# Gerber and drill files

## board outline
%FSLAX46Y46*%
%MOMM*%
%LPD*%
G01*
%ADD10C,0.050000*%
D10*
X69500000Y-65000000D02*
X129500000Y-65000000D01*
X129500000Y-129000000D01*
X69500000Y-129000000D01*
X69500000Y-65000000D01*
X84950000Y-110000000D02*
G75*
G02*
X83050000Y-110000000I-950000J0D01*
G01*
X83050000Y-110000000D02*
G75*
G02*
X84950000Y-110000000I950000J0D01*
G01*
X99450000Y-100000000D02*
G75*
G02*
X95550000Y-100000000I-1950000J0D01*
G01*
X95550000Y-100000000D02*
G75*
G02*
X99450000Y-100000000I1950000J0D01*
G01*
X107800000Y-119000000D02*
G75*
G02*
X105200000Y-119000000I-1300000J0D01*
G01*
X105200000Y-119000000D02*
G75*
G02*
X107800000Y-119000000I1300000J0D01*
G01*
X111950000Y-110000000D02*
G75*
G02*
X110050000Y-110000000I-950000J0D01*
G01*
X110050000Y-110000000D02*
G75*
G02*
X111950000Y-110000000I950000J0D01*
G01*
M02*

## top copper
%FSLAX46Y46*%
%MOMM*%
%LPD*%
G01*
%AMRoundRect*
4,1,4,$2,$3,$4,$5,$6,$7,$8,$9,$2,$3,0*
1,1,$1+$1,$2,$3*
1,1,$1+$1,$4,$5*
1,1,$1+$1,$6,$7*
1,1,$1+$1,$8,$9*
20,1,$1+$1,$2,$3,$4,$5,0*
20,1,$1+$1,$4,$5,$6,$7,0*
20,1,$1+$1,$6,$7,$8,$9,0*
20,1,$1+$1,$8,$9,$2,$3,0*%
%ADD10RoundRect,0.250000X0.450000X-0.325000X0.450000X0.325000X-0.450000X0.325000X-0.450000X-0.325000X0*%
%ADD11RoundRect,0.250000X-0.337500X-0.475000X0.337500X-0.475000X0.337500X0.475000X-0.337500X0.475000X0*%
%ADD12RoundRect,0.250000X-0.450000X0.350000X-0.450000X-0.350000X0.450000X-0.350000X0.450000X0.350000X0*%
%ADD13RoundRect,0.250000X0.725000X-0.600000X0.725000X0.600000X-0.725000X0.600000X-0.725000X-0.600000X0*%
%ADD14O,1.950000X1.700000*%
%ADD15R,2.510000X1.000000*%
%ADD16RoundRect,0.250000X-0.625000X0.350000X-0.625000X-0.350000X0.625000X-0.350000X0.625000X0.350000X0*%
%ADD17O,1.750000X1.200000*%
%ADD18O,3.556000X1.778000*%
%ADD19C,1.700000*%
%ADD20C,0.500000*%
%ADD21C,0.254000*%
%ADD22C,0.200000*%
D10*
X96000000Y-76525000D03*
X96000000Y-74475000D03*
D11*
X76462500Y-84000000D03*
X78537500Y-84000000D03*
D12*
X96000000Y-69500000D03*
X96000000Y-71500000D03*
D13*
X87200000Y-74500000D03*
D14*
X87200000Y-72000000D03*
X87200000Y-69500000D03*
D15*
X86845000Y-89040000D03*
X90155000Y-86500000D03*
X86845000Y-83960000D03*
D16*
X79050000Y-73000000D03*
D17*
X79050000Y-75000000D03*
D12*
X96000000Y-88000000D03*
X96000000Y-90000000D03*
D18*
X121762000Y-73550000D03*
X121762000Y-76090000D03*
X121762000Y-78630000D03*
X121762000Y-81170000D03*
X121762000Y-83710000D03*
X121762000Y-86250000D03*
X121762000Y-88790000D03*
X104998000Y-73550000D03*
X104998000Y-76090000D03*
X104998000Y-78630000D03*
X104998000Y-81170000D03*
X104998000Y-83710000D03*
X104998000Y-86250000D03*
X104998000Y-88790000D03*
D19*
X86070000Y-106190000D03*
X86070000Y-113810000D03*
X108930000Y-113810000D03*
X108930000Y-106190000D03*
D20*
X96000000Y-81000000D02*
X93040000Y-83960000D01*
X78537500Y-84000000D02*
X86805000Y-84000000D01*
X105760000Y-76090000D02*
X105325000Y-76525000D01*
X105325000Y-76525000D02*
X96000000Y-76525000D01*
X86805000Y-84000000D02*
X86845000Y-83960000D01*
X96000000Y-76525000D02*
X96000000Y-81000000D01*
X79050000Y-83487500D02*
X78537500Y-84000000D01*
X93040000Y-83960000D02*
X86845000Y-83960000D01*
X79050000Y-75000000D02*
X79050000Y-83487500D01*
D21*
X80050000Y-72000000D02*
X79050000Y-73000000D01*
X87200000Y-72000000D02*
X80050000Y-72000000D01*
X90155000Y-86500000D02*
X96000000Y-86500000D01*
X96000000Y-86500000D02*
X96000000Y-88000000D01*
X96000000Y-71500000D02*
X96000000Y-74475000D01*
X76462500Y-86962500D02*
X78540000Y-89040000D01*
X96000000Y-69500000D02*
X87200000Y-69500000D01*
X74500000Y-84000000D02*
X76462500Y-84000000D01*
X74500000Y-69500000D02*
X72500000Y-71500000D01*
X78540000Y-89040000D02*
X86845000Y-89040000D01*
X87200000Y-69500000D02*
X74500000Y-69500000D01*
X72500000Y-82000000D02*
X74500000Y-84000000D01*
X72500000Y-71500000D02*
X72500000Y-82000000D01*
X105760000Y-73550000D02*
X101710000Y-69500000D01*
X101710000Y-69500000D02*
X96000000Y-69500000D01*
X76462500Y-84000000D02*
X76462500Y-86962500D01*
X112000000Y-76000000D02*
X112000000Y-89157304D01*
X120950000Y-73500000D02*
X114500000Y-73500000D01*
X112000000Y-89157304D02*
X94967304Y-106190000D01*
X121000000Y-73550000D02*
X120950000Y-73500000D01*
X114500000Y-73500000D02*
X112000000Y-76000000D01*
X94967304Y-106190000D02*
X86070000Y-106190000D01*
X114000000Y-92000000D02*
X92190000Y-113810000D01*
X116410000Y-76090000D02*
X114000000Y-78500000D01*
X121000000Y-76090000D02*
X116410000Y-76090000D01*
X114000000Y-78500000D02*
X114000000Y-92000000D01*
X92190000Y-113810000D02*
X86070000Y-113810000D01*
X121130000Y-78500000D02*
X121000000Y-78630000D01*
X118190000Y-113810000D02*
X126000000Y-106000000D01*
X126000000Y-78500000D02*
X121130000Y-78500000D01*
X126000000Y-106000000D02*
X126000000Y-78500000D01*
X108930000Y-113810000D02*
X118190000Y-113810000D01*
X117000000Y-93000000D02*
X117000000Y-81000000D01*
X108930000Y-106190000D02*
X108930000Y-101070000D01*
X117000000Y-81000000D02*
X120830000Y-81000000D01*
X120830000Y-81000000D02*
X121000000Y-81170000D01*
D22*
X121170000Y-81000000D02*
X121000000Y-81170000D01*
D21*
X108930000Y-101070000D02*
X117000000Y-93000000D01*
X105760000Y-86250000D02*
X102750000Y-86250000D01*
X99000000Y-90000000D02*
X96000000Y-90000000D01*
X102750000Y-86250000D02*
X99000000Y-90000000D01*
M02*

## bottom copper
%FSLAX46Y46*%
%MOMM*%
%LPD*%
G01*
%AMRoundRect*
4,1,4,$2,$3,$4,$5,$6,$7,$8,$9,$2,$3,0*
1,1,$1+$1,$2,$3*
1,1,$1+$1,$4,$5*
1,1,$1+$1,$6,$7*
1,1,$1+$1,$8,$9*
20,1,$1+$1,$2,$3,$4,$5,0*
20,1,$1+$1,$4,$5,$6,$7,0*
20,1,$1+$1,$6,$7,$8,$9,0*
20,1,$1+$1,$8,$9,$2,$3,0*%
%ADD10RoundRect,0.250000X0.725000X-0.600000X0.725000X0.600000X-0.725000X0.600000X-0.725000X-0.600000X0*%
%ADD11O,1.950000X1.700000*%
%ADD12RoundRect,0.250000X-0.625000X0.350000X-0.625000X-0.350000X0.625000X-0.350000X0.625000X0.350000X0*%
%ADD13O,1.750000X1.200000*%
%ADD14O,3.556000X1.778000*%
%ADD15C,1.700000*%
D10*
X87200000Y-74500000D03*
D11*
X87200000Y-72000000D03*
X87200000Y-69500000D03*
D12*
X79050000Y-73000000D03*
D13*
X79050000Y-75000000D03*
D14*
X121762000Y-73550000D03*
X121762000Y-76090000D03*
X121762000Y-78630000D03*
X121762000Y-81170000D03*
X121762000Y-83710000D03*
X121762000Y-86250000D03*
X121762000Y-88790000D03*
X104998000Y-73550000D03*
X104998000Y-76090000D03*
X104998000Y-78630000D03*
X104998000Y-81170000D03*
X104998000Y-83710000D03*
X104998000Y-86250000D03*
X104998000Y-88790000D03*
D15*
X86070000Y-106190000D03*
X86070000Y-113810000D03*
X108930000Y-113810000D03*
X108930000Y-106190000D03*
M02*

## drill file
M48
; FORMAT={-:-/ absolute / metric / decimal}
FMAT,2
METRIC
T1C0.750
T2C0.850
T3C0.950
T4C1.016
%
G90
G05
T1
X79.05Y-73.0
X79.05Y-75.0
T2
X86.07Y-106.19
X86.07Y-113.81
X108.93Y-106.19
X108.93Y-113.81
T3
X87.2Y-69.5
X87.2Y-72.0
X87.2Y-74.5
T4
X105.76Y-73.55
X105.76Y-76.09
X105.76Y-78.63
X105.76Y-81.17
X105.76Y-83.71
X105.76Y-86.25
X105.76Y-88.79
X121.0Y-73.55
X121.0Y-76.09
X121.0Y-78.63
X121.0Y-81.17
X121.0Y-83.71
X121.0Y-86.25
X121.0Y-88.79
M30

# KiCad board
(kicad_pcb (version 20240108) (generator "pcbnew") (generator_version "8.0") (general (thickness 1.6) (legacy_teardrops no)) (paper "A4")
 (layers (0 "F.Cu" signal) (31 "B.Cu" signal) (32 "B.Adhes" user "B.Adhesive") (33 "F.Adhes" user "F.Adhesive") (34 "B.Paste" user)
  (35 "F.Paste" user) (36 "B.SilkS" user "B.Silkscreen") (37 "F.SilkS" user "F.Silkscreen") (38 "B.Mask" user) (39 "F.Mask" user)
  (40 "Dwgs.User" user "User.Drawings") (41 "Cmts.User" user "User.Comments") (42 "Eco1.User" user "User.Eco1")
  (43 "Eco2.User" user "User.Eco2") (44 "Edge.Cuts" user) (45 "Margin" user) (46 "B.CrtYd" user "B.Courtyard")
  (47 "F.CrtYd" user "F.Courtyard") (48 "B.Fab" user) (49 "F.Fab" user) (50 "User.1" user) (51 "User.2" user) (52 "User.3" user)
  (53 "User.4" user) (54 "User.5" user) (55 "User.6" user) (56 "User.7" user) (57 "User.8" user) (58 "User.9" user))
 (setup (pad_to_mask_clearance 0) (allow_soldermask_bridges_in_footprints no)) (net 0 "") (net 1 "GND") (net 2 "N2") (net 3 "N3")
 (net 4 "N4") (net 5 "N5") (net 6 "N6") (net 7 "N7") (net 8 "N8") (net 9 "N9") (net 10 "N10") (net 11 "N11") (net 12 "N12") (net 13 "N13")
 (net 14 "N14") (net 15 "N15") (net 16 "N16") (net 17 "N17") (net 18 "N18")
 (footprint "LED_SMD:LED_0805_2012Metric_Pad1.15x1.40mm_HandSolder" (layer "F.Cu") (at 96 75.5 90)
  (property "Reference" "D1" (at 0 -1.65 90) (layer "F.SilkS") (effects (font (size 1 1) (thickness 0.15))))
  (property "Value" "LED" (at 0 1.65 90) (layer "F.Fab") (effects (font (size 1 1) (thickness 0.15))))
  (pad "1" smd roundrect (at -1.025 0 90) (size 1.15 1.4) (layers "F.Cu" "F.Paste" "F.Mask") (roundrect_rratio 0.217391) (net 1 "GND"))
  (pad "2" smd roundrect (at 1.025 0 90) (size 1.15 1.4) (layers "F.Cu" "F.Paste" "F.Mask") (roundrect_rratio 0.217391) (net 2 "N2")))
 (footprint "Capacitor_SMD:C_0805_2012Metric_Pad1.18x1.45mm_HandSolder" (layer "F.Cu") (at 77.5 84)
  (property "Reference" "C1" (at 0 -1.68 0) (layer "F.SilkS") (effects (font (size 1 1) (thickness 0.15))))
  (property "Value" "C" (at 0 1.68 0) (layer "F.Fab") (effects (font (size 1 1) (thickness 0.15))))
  (pad "1" smd roundrect (at -1.0375 0) (size 1.175 1.45) (layers "F.Cu" "F.Paste" "F.Mask") (roundrect_rratio 0.212766) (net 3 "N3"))
  (pad "2" smd roundrect (at 1.0375 0) (size 1.175 1.45) (layers "F.Cu" "F.Paste" "F.Mask") (roundrect_rratio 0.212766) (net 1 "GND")))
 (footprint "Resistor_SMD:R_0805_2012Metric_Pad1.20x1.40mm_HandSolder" (layer "F.Cu") (at 96 70.5 -90)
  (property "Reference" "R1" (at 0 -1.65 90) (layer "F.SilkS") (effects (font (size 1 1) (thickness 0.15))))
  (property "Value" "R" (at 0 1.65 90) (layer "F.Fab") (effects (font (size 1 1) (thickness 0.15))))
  (pad "1" smd roundrect (at -1 0 270) (size 1.2 1.4) (layers "F.Cu" "F.Paste" "F.Mask") (roundrect_rratio 0.208333) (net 3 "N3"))
  (pad "2" smd roundrect (at 1 0 270) (size 1.2 1.4) (layers "F.Cu" "F.Paste" "F.Mask") (roundrect_rratio 0.208333) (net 2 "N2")))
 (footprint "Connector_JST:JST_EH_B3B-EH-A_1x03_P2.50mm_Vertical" (layer "F.Cu") (at 87.2 74.5 90)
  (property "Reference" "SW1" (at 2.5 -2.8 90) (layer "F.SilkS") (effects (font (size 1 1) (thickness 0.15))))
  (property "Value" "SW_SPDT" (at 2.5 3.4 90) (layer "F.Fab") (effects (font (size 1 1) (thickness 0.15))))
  (pad "1" thru_hole roundrect (at 0 0 90) (size 1.7 1.95) (drill 0.95) (layers "*.Cu" "*.Mask") (remove_unused_layers no)
   (roundrect_rratio 0.147059) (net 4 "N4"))
  (pad "2" thru_hole oval (at 2.5 0 90) (size 1.7 1.95) (drill 0.95) (layers "*.Cu" "*.Mask") (remove_unused_layers no) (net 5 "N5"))
  (pad "3" thru_hole oval (at 5 0 90) (size 1.7 1.95) (drill 0.95) (layers "*.Cu" "*.Mask") (remove_unused_layers no) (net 3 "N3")))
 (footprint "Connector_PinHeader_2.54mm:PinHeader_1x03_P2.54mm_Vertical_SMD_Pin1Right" (layer "F.Cu") (at 88.5 86.5 180)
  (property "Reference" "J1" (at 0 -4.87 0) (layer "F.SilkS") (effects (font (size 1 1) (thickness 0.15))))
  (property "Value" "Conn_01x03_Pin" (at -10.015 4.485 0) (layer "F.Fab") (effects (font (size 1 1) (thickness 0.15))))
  (pad "1" smd rect (at 1.655 -2.54 180) (size 2.51 1) (layers "F.Cu" "F.Paste" "F.Mask") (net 3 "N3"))
  (pad "2" smd rect (at -1.655 0 180) (size 2.51 1) (layers "F.Cu" "F.Paste" "F.Mask") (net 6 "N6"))
  (pad "3" smd rect (at 1.655 2.54 180) (size 2.51 1) (layers "F.Cu" "F.Paste" "F.Mask") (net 1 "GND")))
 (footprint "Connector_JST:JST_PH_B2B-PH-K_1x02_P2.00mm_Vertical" (layer "F.Cu") (at 79.05 73 -90)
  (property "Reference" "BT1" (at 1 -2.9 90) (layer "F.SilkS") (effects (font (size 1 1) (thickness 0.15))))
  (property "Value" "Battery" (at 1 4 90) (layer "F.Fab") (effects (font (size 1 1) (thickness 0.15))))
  (pad "1" thru_hole roundrect (at 0 0 270) (size 1.2 1.75) (drill 0.75) (layers "*.Cu" "*.Mask") (remove_unused_layers no)
   (roundrect_rratio 0.208333) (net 5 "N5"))
  (pad "2" thru_hole oval (at 2 0 270) (size 1.2 1.75) (drill 0.75) (layers "*.Cu" "*.Mask") (remove_unused_layers no) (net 1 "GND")))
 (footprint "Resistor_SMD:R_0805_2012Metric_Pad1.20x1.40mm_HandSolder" (layer "F.Cu") (at 96 89 -90)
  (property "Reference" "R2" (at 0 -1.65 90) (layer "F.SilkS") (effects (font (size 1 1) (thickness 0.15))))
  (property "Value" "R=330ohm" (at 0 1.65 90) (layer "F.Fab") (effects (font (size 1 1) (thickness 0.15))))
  (pad "1" smd roundrect (at -1 0 270) (size 1.2 1.4) (layers "F.Cu" "F.Paste" "F.Mask") (roundrect_rratio 0.208333) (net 6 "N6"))
  (pad "2" smd roundrect (at 1 0 270) (size 1.2 1.4) (layers "F.Cu" "F.Paste" "F.Mask") (roundrect_rratio 0.208333) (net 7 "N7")))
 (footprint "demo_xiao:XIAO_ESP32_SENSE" (layer "B.Cu") (at 113.38 81.17 180)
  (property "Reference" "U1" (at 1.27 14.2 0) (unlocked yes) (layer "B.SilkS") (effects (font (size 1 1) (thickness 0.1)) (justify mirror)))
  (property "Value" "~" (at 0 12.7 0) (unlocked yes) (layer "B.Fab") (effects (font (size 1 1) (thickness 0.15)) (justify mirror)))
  (pad "1" thru_hole oval (at -7.62 7.62 180) (size 3.556 1.778) (drill 1.016 (offset -0.762 0)) (layers "*.Cu" "*.Mask")
   (remove_unused_layers no) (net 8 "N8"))
  (pad "2" thru_hole oval (at -7.62 5.08 180) (size 3.556 1.778) (drill 1.016 (offset -0.762 0)) (layers "*.Cu" "*.Mask")
   (remove_unused_layers no) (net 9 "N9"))
  (pad "3" thru_hole oval (at -7.62 2.54 180) (size 3.556 1.778) (drill 1.016 (offset -0.762 0)) (layers "*.Cu" "*.Mask")
   (remove_unused_layers no) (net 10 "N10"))
  (pad "4" thru_hole oval (at -7.62 0 180) (size 3.556 1.778) (drill 1.016 (offset -0.762 0)) (layers "*.Cu" "*.Mask")
   (remove_unused_layers no) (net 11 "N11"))
  (pad "5" thru_hole oval (at -7.62 -2.54 180) (size 3.556 1.778) (drill 1.016 (offset -0.762 0)) (layers "*.Cu" "*.Mask")
   (remove_unused_layers no) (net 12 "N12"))
  (pad "6" thru_hole oval (at -7.62 -5.08 180) (size 3.556 1.778) (drill 1.016 (offset -0.762 0)) (layers "*.Cu" "*.Mask")
   (remove_unused_layers no) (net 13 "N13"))
  (pad "7" thru_hole oval (at -7.62 -7.62 180) (size 3.556 1.778) (drill 1.016 (offset -0.762 0)) (layers "*.Cu" "*.Mask")
   (remove_unused_layers no) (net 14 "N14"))
  (pad "8" thru_hole oval (at 7.62 7.62 180) (size 3.556 1.778) (drill 1.016 (offset 0.762 0)) (layers "*.Cu" "*.Mask")
   (remove_unused_layers no) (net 3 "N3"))
  (pad "9" thru_hole oval (at 7.62 5.08 180) (size 3.556 1.778) (drill 1.016 (offset 0.762 0)) (layers "*.Cu" "*.Mask")
   (remove_unused_layers no) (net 1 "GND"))
  (pad "10" thru_hole oval (at 7.62 2.54 180) (size 3.556 1.778) (drill 1.016 (offset 0.762 0)) (layers "*.Cu" "*.Mask")
   (remove_unused_layers no) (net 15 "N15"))
  (pad "11" thru_hole oval (at 7.62 0 180) (size 3.556 1.778) (drill 1.016 (offset 0.762 0)) (layers "*.Cu" "*.Mask")
   (remove_unused_layers no) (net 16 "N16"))
  (pad "12" thru_hole oval (at 7.62 -2.54 180) (size 3.556 1.778) (drill 1.016 (offset 0.762 0)) (layers "*.Cu" "*.Mask")
   (remove_unused_layers no) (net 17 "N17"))
  (pad "13" thru_hole oval (at 7.62 -5.08 180) (size 3.556 1.778) (drill 1.016 (offset 0.762 0)) (layers "*.Cu" "*.Mask")
   (remove_unused_layers no) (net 7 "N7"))
  (pad "14" thru_hole oval (at 7.62 -7.62 180) (size 3.556 1.778) (drill 1.016 (offset 0.762 0)) (layers "*.Cu" "*.Mask")
   (remove_unused_layers no) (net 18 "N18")))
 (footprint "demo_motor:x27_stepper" (layer "B.Cu") (at 94.96 120.16 180)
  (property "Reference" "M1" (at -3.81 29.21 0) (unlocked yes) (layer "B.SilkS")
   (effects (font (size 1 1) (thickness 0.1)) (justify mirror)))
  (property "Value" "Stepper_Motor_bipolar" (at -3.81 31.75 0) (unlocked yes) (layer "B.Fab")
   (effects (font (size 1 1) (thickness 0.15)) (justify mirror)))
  (fp_circle (center 10.96 10.16) (end 11.91 10.16) (stroke (width 0.05) (type default)) (fill none) (layer "Edge.Cuts"))
  (fp_circle (center -2.54 20.16) (end -0.59 20.16) (stroke (width 0.05) (type default)) (fill none) (layer "Edge.Cuts"))
  (fp_circle (center -11.54 1.16) (end -10.24 1.16) (stroke (width 0.05) (type default)) (fill none) (layer "Edge.Cuts"))
  (fp_circle (center -16.04 10.16) (end -15.09 10.16) (stroke (width 0.05) (type default)) (fill none) (layer "Edge.Cuts"))
  (pad "1" thru_hole circle (at 8.89 13.97 180) (size 1.7 1.7) (drill 0.85) (layers "*.Cu" "*.Mask") (remove_unused_layers no) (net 8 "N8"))
  (pad "2" thru_hole circle (at 8.89 6.35 180) (size 1.7 1.7) (drill 0.85) (layers "*.Cu" "*.Mask") (remove_unused_layers no) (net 9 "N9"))
  (pad "3" thru_hole circle (at -13.97 6.35 180) (size 1.7 1.7) (drill 0.85) (layers "*.Cu" "*.Mask") (remove_unused_layers no)
   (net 10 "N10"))
  (pad "4" thru_hole circle (at -13.97 13.97 180) (size 1.7 1.7) (drill 0.85) (layers "*.Cu" "*.Mask") (remove_unused_layers no)
   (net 11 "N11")))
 (gr_rect (start 69.5 65) (end 129.5 129) (stroke (width 0.05) (type default)) (fill none) (layer "Edge.Cuts"))
 (segment (start 96 81) (end 93.04 83.96) (width 0.5) (layer "F.Cu") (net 1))
 (segment (start 78.5375 84) (end 86.805 84) (width 0.5) (layer "F.Cu") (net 1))
 (segment (start 105.76 76.09) (end 105.325 76.525) (width 0.5) (layer "F.Cu") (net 1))
 (segment (start 105.325 76.525) (end 96 76.525) (width 0.5) (layer "F.Cu") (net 1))
 (segment (start 86.805 84) (end 86.845 83.96) (width 0.5) (layer "F.Cu") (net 1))
 (segment (start 96 76.525) (end 96 81) (width 0.5) (layer "F.Cu") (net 1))
 (segment (start 79.05 83.4875) (end 78.5375 84) (width 0.5) (layer "F.Cu") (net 1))
 (segment (start 93.04 83.96) (end 86.845 83.96) (width 0.5) (layer "F.Cu") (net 1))
 (segment (start 79.05 75) (end 79.05 83.4875) (width 0.5) (layer "F.Cu") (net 1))
 (segment (start 80.05 72) (end 79.05 73) (width 0.254) (layer "F.Cu") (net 5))
 (segment (start 87.2 72) (end 80.05 72) (width 0.254) (layer "F.Cu") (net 5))
 (segment (start 90.155 86.5) (end 96 86.5) (width 0.254) (layer "F.Cu") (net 6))
 (segment (start 96 86.5) (end 96 88) (width 0.254) (layer "F.Cu") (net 6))
 (segment (start 96 71.5) (end 96 74.475) (width 0.254) (layer "F.Cu") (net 2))
 (segment (start 76.4625 86.9625) (end 78.54 89.04) (width 0.254) (layer "F.Cu") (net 3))
 (segment (start 96 69.5) (end 87.2 69.5) (width 0.254) (layer "F.Cu") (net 3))
 (segment (start 74.5 84) (end 76.4625 84) (width 0.254) (layer "F.Cu") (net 3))
 (segment (start 74.5 69.5) (end 72.5 71.5) (width 0.254) (layer "F.Cu") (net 3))
 (segment (start 78.54 89.04) (end 86.845 89.04) (width 0.254) (layer "F.Cu") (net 3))
 (segment (start 87.2 69.5) (end 74.5 69.5) (width 0.254) (layer "F.Cu") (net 3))
 (segment (start 72.5 82) (end 74.5 84) (width 0.254) (layer "F.Cu") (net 3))
 (segment (start 72.5 71.5) (end 72.5 82) (width 0.254) (layer "F.Cu") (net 3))
 (segment (start 105.76 73.55) (end 101.71 69.5) (width 0.254) (layer "F.Cu") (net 3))
 (segment (start 101.71 69.5) (end 96 69.5) (width 0.254) (layer "F.Cu") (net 3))
 (segment (start 76.4625 84) (end 76.4625 86.9625) (width 0.254) (layer "F.Cu") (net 3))
 (segment (start 112 76) (end 112 89.157304) (width 0.254) (layer "F.Cu") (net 8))
 (segment (start 120.95 73.5) (end 114.5 73.5) (width 0.254) (layer "F.Cu") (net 8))
 (segment (start 112 89.157304) (end 94.967304 106.19) (width 0.254) (layer "F.Cu") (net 8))
 (segment (start 121 73.55) (end 120.95 73.5) (width 0.254) (layer "F.Cu") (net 8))
 (segment (start 114.5 73.5) (end 112 76) (width 0.254) (layer "F.Cu") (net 8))
 (segment (start 94.967304 106.19) (end 86.07 106.19) (width 0.254) (layer "F.Cu") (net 8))
 (segment (start 114 92) (end 92.19 113.81) (width 0.254) (layer "F.Cu") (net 9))
 (segment (start 116.41 76.09) (end 114 78.5) (width 0.254) (layer "F.Cu") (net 9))
 (segment (start 121 76.09) (end 116.41 76.09) (width 0.254) (layer "F.Cu") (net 9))
 (segment (start 114 78.5) (end 114 92) (width 0.254) (layer "F.Cu") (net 9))
 (segment (start 92.19 113.81) (end 86.07 113.81) (width 0.254) (layer "F.Cu") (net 9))
 (segment (start 121.13 78.5) (end 121 78.63) (width 0.254) (layer "F.Cu") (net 10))
 (segment (start 118.19 113.81) (end 126 106) (width 0.254) (layer "F.Cu") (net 10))
 (segment (start 126 78.5) (end 121.13 78.5) (width 0.254) (layer "F.Cu") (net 10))
 (segment (start 126 106) (end 126 78.5) (width 0.254) (layer "F.Cu") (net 10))
 (segment (start 108.93 113.81) (end 118.19 113.81) (width 0.254) (layer "F.Cu") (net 10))
 (segment (start 117 93) (end 117 81) (width 0.254) (layer "F.Cu") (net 11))
 (segment (start 108.93 106.19) (end 108.93 101.07) (width 0.254) (layer "F.Cu") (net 11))
 (segment (start 117 81) (end 120.83 81) (width 0.254) (layer "F.Cu") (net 11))
 (segment (start 120.83 81) (end 121 81.17) (width 0.254) (layer "F.Cu") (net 11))
 (segment (start 121.17 81) (end 121 81.17) (width 0.2) (layer "F.Cu") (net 11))
 (segment (start 108.93 101.07) (end 117 93) (width 0.254) (layer "F.Cu") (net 11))
 (segment (start 105.76 86.25) (end 102.75 86.25) (width 0.254) (layer "F.Cu") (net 7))
 (segment (start 99 90) (end 96 90) (width 0.254) (layer "F.Cu") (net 7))
 (segment (start 102.75 86.25) (end 99 90) (width 0.254) (layer "F.Cu") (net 7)))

